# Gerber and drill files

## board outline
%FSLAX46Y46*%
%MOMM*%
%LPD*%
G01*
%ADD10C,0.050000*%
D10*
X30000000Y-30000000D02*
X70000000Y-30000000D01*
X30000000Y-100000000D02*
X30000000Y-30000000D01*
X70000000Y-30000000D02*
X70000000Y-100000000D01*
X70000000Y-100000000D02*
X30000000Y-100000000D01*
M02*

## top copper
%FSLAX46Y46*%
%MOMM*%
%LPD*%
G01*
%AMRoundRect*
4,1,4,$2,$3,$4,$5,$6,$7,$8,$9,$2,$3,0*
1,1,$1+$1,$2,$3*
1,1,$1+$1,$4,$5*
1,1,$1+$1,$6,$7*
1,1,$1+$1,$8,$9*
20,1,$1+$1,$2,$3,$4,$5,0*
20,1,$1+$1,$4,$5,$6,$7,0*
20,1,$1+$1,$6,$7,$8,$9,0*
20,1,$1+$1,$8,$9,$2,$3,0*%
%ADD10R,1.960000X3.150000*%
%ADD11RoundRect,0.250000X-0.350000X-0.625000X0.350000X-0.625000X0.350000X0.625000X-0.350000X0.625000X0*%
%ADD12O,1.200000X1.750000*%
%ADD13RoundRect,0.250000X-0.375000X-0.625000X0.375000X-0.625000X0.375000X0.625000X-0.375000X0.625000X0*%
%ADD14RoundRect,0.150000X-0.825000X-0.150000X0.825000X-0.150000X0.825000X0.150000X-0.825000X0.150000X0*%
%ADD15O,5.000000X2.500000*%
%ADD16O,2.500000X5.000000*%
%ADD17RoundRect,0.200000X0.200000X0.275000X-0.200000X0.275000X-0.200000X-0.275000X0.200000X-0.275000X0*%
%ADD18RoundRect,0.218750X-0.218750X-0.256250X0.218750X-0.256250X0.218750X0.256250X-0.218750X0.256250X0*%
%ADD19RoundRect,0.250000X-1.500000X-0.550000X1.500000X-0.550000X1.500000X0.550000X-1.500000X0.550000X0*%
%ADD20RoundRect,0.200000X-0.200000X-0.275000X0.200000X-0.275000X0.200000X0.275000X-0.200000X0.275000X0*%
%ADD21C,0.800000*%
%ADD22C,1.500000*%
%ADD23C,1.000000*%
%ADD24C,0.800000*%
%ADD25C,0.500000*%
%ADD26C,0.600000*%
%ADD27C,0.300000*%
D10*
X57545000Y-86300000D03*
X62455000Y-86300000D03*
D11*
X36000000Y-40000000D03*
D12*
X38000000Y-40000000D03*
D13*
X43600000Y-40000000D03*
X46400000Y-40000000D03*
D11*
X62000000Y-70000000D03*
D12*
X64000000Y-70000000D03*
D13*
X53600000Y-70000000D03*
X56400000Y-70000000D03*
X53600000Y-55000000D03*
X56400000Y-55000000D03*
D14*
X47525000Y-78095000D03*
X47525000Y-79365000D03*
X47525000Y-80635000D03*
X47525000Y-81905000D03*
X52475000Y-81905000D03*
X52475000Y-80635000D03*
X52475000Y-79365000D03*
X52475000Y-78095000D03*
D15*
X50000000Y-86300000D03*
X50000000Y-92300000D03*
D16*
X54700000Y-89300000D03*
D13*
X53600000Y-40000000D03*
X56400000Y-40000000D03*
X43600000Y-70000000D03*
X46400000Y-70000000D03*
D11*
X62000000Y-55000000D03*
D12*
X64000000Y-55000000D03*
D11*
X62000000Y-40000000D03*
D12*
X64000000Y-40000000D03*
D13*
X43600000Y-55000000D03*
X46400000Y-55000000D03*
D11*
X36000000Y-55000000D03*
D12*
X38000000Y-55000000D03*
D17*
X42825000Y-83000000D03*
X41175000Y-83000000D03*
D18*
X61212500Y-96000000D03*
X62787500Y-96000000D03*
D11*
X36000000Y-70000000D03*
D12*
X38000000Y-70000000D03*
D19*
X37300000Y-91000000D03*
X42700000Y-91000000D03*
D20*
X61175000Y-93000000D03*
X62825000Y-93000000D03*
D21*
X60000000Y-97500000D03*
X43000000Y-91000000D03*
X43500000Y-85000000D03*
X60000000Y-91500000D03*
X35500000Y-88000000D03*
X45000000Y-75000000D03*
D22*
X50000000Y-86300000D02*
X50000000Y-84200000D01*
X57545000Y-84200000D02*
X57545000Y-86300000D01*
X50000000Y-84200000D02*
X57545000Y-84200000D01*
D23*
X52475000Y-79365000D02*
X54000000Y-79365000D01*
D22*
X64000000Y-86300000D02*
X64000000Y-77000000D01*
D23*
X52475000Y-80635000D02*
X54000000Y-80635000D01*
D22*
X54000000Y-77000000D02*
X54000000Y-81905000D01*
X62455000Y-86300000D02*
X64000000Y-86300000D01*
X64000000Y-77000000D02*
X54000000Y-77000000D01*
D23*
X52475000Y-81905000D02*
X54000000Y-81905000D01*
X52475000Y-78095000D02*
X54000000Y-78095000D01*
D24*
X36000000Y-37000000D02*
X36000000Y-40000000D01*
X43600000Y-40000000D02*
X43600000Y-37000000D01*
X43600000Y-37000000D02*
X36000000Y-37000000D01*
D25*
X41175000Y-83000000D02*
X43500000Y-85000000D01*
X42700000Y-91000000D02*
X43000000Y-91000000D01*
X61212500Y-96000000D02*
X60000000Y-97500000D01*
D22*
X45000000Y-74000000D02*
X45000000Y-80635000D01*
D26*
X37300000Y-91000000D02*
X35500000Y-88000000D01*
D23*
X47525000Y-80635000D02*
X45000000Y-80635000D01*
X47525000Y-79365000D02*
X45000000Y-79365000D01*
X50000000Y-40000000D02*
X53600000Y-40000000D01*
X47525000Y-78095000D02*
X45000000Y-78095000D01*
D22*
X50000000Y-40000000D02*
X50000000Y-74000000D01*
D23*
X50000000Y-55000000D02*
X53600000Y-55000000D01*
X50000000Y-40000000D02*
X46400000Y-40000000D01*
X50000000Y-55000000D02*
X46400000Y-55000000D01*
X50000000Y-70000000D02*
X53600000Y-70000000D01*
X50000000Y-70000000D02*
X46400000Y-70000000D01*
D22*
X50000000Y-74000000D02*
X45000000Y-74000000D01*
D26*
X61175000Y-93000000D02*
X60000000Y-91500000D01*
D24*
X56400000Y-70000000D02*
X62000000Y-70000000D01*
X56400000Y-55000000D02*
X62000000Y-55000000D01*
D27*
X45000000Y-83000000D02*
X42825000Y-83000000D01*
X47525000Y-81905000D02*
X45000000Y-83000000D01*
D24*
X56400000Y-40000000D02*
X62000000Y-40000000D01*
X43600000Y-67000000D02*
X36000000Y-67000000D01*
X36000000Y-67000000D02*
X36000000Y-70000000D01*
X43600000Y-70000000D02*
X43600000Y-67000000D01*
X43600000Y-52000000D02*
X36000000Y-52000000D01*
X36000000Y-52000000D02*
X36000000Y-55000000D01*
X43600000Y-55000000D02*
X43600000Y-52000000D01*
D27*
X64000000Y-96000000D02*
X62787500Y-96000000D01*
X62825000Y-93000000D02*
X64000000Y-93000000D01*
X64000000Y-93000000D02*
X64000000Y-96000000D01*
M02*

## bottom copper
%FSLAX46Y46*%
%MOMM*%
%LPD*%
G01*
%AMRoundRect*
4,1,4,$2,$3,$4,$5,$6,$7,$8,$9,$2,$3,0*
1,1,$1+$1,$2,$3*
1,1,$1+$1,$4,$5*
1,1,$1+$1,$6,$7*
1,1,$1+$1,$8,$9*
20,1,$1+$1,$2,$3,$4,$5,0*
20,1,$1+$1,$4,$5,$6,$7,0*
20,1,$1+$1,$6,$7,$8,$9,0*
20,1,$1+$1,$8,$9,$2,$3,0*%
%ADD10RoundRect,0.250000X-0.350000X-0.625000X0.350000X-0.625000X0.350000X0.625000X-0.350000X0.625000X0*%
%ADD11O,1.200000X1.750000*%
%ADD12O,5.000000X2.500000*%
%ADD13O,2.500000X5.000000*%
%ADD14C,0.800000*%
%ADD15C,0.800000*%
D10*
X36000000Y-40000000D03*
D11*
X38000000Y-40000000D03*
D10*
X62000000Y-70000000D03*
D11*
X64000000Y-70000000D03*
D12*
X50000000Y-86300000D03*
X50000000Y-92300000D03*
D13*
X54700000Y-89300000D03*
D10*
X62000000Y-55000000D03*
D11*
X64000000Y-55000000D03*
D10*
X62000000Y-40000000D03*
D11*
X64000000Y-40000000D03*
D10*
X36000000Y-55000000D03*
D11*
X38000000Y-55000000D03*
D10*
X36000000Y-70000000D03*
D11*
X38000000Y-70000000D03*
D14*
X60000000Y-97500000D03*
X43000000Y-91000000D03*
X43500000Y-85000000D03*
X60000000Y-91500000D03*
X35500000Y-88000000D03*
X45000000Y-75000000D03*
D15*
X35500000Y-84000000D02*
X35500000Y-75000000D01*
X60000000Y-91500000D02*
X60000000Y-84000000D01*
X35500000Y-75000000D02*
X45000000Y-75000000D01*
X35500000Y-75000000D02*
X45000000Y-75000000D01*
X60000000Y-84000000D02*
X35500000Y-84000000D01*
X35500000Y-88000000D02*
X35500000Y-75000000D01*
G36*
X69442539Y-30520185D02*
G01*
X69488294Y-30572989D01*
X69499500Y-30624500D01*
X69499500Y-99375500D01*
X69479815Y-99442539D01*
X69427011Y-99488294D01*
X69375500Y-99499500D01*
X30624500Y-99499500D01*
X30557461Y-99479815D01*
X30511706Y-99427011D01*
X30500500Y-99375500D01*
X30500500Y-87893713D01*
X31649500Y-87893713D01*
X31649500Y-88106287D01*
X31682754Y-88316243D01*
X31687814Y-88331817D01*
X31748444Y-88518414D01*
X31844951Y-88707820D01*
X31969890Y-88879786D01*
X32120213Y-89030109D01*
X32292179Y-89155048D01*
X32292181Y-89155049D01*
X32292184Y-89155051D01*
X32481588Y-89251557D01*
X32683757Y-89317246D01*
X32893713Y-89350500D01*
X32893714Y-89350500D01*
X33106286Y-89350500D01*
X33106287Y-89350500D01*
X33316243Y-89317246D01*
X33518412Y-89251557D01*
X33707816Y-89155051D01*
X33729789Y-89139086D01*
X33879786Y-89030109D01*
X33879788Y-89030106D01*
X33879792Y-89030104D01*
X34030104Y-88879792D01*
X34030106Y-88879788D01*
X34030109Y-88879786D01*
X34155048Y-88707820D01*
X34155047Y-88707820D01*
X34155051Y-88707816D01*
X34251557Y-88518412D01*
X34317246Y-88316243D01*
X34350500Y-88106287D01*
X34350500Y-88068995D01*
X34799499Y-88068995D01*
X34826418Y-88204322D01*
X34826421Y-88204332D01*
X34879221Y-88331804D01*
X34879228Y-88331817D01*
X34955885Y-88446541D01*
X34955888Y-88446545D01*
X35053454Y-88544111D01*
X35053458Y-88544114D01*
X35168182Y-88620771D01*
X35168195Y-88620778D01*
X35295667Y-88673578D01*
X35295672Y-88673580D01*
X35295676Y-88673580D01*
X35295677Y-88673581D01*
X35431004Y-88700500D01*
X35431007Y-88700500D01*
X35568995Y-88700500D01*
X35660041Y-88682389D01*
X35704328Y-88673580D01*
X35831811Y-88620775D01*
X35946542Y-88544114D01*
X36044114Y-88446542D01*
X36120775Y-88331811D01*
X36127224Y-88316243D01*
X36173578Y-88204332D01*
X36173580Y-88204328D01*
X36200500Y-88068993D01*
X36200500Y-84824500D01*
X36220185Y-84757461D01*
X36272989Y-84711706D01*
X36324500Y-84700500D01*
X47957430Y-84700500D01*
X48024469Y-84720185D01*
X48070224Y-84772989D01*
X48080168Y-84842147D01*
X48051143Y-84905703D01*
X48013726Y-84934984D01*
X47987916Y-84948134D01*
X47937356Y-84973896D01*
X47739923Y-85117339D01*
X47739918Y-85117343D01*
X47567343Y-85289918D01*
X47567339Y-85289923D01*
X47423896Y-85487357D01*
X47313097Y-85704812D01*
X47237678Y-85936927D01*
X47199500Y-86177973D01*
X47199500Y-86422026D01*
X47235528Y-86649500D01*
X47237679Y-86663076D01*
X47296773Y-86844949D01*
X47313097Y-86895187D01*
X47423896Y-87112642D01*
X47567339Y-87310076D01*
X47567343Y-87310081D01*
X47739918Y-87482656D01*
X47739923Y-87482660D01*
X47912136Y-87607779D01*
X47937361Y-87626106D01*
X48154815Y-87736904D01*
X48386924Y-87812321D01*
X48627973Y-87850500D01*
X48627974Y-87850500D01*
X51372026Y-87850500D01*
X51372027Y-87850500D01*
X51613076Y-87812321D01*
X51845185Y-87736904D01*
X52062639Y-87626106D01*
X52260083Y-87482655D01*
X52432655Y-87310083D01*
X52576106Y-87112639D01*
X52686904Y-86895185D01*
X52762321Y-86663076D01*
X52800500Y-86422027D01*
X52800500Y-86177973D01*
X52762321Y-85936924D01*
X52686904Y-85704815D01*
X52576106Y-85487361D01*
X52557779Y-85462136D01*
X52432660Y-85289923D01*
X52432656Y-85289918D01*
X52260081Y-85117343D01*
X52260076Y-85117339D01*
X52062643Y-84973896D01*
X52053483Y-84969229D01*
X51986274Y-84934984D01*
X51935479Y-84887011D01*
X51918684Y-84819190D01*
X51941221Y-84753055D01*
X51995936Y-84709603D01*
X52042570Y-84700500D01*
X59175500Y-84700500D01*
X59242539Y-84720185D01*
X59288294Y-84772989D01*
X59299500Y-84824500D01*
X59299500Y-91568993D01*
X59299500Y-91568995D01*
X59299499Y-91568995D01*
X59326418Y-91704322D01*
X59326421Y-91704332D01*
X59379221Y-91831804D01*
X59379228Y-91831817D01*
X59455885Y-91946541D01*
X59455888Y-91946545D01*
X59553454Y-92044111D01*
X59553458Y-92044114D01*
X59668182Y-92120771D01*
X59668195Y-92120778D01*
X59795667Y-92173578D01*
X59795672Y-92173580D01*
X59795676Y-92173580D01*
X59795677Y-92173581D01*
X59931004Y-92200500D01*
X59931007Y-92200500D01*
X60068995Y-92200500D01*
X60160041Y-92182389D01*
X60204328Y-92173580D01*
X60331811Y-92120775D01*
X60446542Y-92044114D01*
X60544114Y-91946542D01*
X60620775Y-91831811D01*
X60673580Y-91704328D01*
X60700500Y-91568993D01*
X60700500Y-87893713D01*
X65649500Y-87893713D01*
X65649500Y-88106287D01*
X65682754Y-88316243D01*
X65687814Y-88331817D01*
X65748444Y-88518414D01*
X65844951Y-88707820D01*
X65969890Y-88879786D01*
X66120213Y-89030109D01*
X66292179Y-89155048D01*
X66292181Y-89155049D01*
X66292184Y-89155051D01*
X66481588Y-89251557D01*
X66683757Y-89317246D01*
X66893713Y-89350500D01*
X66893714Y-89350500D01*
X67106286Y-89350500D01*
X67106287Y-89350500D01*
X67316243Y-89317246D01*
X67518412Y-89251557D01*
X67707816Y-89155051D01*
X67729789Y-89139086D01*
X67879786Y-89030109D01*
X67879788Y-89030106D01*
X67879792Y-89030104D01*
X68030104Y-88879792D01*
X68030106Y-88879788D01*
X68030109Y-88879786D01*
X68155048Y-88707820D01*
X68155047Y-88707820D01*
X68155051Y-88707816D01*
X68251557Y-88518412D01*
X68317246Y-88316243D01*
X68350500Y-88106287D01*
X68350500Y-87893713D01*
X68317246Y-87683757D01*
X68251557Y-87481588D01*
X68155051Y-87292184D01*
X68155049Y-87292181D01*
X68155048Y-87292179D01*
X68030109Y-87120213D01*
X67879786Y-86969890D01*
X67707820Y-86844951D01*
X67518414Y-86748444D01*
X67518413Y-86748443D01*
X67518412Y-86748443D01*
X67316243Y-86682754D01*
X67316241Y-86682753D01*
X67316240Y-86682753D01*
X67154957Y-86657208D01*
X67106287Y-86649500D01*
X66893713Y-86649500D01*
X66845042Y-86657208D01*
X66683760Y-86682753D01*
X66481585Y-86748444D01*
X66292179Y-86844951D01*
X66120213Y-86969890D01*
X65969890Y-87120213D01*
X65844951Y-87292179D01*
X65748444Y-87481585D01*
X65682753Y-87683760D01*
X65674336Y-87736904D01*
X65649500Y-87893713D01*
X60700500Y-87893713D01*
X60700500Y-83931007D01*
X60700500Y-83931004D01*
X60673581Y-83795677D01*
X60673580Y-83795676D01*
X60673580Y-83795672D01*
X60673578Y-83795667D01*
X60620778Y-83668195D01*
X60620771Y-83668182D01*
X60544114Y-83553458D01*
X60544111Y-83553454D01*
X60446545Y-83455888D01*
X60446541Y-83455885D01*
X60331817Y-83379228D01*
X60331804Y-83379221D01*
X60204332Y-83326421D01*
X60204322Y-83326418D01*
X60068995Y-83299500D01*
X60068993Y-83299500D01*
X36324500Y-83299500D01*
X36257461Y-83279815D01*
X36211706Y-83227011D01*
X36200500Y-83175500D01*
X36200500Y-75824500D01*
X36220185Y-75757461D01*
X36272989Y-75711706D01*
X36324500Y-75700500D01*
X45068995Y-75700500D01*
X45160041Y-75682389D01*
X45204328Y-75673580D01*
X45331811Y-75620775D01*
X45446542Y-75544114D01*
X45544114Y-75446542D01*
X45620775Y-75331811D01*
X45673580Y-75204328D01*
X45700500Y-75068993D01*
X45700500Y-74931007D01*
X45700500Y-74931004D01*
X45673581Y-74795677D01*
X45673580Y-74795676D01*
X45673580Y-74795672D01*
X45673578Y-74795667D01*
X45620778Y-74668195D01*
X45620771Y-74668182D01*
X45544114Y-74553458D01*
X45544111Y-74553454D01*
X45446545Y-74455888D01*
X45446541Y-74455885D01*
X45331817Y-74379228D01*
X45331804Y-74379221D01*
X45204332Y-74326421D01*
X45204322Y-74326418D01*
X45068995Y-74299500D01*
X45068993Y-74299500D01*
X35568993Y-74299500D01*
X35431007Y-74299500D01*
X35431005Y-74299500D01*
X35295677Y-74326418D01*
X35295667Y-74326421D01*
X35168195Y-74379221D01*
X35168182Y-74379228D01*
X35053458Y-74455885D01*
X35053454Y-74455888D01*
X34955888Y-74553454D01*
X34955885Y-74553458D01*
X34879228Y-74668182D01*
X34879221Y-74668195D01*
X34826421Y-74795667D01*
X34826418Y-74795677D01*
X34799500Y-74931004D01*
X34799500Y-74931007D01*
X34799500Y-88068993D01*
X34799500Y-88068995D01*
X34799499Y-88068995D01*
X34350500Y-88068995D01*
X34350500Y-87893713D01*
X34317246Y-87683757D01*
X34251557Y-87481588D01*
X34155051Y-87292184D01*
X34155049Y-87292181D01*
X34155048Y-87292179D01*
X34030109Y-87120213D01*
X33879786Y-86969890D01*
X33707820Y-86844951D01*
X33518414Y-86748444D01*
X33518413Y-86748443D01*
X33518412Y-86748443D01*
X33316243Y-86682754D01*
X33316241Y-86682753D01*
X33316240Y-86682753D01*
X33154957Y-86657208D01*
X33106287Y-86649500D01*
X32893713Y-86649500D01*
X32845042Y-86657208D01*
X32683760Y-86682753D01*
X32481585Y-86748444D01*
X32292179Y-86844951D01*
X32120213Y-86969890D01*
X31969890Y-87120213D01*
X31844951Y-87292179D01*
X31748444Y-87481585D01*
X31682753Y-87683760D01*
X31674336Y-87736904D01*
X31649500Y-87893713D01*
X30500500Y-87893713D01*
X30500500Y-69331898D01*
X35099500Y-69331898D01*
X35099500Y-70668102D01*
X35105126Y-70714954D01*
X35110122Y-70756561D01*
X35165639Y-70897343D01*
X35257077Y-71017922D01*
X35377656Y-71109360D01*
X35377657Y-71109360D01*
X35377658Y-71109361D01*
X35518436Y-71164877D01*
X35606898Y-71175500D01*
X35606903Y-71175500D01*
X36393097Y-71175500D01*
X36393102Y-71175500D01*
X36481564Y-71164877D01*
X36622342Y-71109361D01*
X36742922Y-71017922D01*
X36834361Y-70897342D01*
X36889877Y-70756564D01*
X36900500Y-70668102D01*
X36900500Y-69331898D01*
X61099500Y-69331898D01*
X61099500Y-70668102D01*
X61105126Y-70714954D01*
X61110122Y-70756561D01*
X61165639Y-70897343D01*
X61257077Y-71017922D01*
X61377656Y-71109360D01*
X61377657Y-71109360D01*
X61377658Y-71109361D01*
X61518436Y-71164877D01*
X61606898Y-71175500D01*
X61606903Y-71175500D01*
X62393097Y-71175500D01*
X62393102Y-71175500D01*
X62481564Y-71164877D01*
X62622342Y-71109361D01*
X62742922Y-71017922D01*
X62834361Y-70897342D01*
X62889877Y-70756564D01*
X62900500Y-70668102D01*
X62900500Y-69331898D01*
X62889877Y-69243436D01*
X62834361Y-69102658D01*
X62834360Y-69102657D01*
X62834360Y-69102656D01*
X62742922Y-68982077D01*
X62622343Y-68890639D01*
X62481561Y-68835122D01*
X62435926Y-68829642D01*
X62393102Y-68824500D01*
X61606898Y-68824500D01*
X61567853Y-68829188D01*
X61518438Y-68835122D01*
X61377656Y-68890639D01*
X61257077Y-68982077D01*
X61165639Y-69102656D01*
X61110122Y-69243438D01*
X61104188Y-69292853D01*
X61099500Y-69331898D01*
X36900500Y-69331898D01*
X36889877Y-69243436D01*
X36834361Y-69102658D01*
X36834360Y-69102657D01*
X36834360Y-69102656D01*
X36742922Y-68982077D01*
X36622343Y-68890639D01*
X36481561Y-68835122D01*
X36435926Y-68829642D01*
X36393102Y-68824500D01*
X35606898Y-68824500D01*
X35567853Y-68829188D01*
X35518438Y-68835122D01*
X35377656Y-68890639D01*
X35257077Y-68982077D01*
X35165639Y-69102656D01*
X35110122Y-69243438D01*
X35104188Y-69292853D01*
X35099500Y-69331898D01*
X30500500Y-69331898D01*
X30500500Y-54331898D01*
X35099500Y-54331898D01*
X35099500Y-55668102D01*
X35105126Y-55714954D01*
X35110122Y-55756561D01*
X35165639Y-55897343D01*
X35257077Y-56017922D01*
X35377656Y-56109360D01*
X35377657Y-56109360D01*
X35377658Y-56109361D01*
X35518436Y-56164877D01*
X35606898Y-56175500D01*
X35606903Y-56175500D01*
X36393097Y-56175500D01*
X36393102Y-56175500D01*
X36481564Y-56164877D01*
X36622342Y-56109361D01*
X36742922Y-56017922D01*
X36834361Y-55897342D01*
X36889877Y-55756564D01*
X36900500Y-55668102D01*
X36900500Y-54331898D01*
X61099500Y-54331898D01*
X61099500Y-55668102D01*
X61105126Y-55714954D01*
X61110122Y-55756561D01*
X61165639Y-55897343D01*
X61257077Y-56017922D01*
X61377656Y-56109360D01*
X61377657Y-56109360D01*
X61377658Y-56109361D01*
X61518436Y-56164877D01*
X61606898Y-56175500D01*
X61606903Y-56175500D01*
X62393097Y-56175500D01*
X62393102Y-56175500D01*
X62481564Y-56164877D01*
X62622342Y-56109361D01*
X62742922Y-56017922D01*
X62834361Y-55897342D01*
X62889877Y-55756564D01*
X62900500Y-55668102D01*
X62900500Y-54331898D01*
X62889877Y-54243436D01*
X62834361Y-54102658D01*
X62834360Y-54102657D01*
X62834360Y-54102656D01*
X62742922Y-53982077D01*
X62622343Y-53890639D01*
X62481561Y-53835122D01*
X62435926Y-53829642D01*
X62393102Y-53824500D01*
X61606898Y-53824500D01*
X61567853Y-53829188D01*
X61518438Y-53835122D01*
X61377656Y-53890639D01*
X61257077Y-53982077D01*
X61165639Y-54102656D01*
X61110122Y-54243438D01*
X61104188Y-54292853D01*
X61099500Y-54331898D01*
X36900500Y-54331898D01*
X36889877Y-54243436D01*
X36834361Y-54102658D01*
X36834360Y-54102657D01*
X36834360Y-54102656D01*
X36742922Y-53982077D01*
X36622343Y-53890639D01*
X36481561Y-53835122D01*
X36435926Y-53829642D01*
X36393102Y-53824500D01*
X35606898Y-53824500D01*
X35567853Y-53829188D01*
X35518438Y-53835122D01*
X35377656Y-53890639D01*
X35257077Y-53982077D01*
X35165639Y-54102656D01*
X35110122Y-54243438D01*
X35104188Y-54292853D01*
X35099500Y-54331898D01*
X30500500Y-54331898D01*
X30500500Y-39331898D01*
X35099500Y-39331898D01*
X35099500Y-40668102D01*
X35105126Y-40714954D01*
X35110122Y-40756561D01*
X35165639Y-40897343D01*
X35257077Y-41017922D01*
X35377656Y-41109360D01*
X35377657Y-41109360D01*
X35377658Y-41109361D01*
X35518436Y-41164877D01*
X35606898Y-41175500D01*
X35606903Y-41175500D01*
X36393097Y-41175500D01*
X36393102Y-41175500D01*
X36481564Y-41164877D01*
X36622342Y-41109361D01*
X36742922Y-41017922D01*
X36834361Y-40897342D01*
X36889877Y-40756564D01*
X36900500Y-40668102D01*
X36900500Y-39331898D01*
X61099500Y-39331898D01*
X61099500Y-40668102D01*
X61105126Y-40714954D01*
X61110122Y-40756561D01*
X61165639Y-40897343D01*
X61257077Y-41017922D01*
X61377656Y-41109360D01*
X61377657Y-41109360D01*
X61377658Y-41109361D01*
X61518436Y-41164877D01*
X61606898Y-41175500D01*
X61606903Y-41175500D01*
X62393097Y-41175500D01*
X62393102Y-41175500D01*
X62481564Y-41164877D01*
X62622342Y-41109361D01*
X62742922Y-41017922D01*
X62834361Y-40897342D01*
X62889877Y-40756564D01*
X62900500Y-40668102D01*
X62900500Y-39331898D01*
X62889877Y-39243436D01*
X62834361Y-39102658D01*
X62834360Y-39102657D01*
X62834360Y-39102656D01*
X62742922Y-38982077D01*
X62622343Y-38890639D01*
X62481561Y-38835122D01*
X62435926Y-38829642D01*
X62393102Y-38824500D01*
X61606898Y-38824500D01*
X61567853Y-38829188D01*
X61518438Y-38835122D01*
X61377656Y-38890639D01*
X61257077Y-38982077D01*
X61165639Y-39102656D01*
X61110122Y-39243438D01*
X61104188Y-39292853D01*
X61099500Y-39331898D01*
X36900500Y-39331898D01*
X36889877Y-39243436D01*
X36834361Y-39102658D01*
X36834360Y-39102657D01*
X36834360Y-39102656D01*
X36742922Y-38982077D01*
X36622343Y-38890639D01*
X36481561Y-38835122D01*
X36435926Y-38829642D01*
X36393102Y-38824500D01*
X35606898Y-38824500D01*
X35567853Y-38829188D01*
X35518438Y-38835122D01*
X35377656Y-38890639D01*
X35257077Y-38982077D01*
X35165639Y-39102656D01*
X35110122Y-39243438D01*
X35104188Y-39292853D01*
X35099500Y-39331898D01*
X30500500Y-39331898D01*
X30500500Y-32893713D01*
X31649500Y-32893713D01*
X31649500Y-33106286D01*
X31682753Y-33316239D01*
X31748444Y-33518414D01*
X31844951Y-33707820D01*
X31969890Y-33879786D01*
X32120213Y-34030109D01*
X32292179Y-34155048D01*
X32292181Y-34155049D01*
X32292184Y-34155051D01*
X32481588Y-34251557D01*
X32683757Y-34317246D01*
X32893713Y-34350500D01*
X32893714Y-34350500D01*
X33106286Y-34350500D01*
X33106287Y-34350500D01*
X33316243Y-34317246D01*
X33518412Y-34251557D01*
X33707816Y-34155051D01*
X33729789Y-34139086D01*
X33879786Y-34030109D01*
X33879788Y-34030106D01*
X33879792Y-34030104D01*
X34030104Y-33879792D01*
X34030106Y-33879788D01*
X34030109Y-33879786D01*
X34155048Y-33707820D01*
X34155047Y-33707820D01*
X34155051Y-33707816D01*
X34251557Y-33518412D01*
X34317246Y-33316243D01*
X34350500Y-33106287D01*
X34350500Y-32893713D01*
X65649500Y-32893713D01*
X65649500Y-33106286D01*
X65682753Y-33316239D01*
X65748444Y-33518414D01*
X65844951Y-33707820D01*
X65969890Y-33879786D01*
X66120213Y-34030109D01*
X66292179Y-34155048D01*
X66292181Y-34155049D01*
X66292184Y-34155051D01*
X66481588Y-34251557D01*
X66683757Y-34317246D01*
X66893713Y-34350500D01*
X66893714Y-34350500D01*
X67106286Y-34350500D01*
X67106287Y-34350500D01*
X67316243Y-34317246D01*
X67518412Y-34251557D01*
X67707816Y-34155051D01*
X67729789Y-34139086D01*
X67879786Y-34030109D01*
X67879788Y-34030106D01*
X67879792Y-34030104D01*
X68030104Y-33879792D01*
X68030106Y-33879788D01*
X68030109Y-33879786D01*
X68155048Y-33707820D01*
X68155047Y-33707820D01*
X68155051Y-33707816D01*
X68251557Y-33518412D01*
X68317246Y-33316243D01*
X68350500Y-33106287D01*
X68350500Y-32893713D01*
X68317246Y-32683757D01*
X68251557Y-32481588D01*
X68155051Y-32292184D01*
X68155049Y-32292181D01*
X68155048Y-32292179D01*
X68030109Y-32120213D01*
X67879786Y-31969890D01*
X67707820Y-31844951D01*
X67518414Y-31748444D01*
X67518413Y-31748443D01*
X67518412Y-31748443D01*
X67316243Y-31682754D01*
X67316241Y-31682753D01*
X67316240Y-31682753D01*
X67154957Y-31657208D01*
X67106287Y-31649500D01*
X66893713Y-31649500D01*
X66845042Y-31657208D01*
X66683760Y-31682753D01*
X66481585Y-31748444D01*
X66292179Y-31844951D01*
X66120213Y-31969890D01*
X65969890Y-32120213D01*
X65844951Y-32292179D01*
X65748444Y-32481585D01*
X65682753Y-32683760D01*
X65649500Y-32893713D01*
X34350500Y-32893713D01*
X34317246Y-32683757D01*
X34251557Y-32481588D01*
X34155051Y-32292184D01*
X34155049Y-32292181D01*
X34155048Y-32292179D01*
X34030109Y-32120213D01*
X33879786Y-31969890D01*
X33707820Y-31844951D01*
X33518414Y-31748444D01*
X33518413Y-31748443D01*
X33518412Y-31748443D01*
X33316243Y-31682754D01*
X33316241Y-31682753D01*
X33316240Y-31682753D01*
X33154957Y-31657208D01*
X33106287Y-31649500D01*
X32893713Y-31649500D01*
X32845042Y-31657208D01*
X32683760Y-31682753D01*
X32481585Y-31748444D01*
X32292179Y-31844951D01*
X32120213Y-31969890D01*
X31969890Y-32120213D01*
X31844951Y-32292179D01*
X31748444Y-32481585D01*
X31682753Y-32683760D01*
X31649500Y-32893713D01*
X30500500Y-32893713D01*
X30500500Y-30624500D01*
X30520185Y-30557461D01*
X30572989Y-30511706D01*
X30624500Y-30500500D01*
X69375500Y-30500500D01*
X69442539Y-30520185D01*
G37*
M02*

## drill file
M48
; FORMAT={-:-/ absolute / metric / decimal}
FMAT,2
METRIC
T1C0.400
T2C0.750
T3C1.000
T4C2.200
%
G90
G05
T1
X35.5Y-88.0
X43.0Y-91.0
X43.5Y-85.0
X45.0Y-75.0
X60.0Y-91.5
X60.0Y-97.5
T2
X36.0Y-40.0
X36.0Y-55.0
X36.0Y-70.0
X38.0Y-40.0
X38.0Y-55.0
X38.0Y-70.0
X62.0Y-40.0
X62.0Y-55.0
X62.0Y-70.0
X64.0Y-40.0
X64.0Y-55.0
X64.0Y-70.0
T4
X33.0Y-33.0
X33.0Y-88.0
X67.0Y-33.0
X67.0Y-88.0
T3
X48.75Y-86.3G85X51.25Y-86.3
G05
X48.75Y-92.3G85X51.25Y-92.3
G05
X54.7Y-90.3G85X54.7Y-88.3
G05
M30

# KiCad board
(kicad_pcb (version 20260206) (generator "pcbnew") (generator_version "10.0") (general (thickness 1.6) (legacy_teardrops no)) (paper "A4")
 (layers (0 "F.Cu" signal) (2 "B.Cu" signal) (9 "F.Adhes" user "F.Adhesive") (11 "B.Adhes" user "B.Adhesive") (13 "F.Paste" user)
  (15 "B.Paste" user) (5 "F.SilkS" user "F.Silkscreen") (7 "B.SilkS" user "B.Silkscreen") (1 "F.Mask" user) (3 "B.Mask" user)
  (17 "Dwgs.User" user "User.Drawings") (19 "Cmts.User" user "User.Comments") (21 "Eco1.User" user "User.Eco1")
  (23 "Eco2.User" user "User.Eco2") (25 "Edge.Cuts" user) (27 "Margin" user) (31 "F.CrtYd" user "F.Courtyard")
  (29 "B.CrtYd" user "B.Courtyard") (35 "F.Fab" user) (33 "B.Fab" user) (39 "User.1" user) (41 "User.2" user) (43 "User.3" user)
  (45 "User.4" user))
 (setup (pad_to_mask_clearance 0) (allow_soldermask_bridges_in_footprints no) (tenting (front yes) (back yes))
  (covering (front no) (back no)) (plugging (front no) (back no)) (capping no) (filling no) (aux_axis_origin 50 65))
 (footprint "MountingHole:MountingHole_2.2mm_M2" (layer "F.Cu") (at 33 88)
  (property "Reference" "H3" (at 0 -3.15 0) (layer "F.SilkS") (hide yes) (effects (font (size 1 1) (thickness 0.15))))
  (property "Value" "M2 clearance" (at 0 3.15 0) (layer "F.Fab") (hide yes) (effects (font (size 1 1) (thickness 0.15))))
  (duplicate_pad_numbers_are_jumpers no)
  (pad "" np_thru_hole circle (at 0 0) (size 2.2 2.2) (drill 2.2) (layers "*.Cu" "*.Mask")))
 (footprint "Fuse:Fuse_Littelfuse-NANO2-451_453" (layer "F.Cu") (at 60 86.3)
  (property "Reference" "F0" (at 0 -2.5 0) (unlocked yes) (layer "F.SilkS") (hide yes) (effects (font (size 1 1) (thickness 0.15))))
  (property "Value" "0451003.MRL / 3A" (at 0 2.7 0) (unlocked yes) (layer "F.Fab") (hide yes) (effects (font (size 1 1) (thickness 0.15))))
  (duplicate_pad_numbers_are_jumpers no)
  (pad "1" smd rect (at -2.455 0) (size 1.96 3.15) (layers "F.Cu" "F.Mask" "F.Paste") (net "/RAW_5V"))
  (pad "2" smd rect (at 2.455 0) (size 1.96 3.15) (layers "F.Cu" "F.Mask" "F.Paste") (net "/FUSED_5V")))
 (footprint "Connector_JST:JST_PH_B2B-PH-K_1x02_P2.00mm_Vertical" (layer "F.Cu") (at 36 40)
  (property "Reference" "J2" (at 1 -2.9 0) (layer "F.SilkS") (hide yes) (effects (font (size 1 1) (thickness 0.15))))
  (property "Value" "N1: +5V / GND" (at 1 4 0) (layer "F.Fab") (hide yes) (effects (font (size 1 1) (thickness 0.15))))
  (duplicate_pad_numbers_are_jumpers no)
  (pad "1" thru_hole roundrect (at 0 0) (size 1.2 1.75) (drill 0.75) (layers "*.Cu" "*.Mask") (remove_unused_layers no)
   (roundrect_rratio 0.208333) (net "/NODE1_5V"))
  (pad "2" thru_hole oval (at 2 0) (size 1.2 1.75) (drill 0.75) (layers "*.Cu" "*.Mask") (remove_unused_layers no) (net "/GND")))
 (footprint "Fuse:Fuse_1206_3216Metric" (layer "F.Cu") (at 45 40)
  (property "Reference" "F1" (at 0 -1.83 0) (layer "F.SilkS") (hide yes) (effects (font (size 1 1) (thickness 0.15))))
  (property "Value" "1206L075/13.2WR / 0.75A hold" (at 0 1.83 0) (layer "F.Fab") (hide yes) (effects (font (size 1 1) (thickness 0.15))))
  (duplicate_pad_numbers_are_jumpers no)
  (pad "1" smd roundrect (at -1.4 0) (size 1.25 1.75) (layers "F.Cu" "F.Mask" "F.Paste") (roundrect_rratio 0.2) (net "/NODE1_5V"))
  (pad "2" smd roundrect (at 1.4 0) (size 1.25 1.75) (layers "F.Cu" "F.Mask" "F.Paste") (roundrect_rratio 0.2) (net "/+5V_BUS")))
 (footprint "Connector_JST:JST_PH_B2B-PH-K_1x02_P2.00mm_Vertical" (layer "F.Cu") (at 62 70)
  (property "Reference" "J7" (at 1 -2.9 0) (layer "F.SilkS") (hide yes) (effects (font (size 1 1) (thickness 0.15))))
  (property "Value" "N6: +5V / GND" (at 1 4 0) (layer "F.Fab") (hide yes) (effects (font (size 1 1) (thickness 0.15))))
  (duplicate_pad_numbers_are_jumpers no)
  (pad "1" thru_hole roundrect (at 0 0) (size 1.2 1.75) (drill 0.75) (layers "*.Cu" "*.Mask") (remove_unused_layers no)
   (roundrect_rratio 0.208333) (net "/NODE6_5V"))
  (pad "2" thru_hole oval (at 2 0) (size 1.2 1.75) (drill 0.75) (layers "*.Cu" "*.Mask") (remove_unused_layers no) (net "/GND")))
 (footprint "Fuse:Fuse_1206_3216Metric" (layer "F.Cu") (at 55 70)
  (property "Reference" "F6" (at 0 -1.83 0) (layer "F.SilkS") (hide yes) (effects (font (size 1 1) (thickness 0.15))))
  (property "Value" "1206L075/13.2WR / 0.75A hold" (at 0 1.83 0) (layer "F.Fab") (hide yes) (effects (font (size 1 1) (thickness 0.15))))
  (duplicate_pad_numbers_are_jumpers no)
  (pad "1" smd roundrect (at -1.4 0) (size 1.25 1.75) (layers "F.Cu" "F.Mask" "F.Paste") (roundrect_rratio 0.2) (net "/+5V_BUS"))
  (pad "2" smd roundrect (at 1.4 0) (size 1.25 1.75) (layers "F.Cu" "F.Mask" "F.Paste") (roundrect_rratio 0.2) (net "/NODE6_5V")))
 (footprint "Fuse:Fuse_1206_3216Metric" (layer "F.Cu") (at 55 55)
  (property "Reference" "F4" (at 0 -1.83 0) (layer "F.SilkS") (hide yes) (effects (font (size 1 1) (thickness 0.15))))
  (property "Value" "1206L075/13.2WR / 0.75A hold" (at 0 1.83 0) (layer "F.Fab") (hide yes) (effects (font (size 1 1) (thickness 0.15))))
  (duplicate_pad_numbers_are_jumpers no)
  (pad "1" smd roundrect (at -1.4 0) (size 1.25 1.75) (layers "F.Cu" "F.Mask" "F.Paste") (roundrect_rratio 0.2) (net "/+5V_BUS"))
  (pad "2" smd roundrect (at 1.4 0) (size 1.25 1.75) (layers "F.Cu" "F.Mask" "F.Paste") (roundrect_rratio 0.2) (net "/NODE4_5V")))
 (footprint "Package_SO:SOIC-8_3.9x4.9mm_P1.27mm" (layer "F.Cu") (at 50 80)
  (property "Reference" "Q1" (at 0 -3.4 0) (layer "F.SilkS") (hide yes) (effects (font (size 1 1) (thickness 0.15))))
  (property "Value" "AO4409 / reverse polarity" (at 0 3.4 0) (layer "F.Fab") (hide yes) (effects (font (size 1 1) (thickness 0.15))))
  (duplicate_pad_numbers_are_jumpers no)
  (pad "1" smd roundrect (at -2.475 -1.905) (size 1.95 0.6) (layers "F.Cu" "F.Mask" "F.Paste") (roundrect_rratio 0.25) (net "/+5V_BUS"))
  (pad "2" smd roundrect (at -2.475 -0.635) (size 1.95 0.6) (layers "F.Cu" "F.Mask" "F.Paste") (roundrect_rratio 0.25) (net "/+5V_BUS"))
  (pad "3" smd roundrect (at -2.475 0.635) (size 1.95 0.6) (layers "F.Cu" "F.Mask" "F.Paste") (roundrect_rratio 0.25) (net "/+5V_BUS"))
  (pad "4" smd roundrect (at -2.475 1.905) (size 1.95 0.6) (layers "F.Cu" "F.Mask" "F.Paste") (roundrect_rratio 0.25) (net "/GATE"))
  (pad "5" smd roundrect (at 2.475 1.905) (size 1.95 0.6) (layers "F.Cu" "F.Mask" "F.Paste") (roundrect_rratio 0.25) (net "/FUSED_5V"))
  (pad "6" smd roundrect (at 2.475 0.635) (size 1.95 0.6) (layers "F.Cu" "F.Mask" "F.Paste") (roundrect_rratio 0.25) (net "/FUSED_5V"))
  (pad "7" smd roundrect (at 2.475 -0.635) (size 1.95 0.6) (layers "F.Cu" "F.Mask" "F.Paste") (roundrect_rratio 0.25) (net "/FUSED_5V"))
  (pad "8" smd roundrect (at 2.475 -1.905) (size 1.95 0.6) (layers "F.Cu" "F.Mask" "F.Paste") (roundrect_rratio 0.25) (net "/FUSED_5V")))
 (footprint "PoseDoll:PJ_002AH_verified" (layer "F.Cu") (at 50 86.3 90)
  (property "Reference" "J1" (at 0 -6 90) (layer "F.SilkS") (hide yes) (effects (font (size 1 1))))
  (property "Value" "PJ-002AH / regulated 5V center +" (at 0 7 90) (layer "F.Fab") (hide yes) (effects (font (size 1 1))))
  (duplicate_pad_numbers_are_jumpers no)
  (pad "1" thru_hole oval (at 0 0 90) (size 2.5 5) (drill oval 1 3.5) (layers "*.Cu" "*.Mask") (remove_unused_layers no) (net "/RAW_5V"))
  (pad "2" thru_hole oval (at -6 0 90) (size 2.5 5) (drill oval 1 3.5) (layers "*.Cu" "*.Mask") (remove_unused_layers no) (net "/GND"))
  (pad "3" thru_hole oval (at -3 4.7 90) (size 5 2.5) (drill oval 3 1) (layers "*.Cu" "*.Mask") (remove_unused_layers no) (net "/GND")))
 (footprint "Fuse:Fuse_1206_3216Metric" (layer "F.Cu") (at 55 40)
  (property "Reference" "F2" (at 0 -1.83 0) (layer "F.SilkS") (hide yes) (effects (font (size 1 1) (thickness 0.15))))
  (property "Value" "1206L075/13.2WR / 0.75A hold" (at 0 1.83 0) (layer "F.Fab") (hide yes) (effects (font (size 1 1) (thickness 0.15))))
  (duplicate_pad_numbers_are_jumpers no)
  (pad "1" smd roundrect (at -1.4 0) (size 1.25 1.75) (layers "F.Cu" "F.Mask" "F.Paste") (roundrect_rratio 0.2) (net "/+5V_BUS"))
  (pad "2" smd roundrect (at 1.4 0) (size 1.25 1.75) (layers "F.Cu" "F.Mask" "F.Paste") (roundrect_rratio 0.2) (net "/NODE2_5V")))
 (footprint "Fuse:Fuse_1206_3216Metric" (layer "F.Cu") (at 45 70)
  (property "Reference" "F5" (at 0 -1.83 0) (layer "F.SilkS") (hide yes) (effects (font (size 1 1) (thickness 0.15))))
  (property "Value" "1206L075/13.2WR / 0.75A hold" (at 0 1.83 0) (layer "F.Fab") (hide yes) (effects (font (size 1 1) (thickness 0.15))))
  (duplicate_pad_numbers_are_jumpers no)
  (pad "1" smd roundrect (at -1.4 0) (size 1.25 1.75) (layers "F.Cu" "F.Mask" "F.Paste") (roundrect_rratio 0.2) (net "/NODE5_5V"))
  (pad "2" smd roundrect (at 1.4 0) (size 1.25 1.75) (layers "F.Cu" "F.Mask" "F.Paste") (roundrect_rratio 0.2) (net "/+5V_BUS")))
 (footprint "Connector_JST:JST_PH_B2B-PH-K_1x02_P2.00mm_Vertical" (layer "F.Cu") (at 62 55)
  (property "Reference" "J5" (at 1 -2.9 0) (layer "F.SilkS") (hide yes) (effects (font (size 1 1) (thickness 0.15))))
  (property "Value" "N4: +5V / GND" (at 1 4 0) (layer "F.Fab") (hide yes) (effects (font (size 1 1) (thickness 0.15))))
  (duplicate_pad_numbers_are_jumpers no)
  (pad "1" thru_hole roundrect (at 0 0) (size 1.2 1.75) (drill 0.75) (layers "*.Cu" "*.Mask") (remove_unused_layers no)
   (roundrect_rratio 0.208333) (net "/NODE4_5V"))
  (pad "2" thru_hole oval (at 2 0) (size 1.2 1.75) (drill 0.75) (layers "*.Cu" "*.Mask") (remove_unused_layers no) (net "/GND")))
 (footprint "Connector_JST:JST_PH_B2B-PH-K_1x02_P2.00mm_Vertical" (layer "F.Cu") (at 62 40)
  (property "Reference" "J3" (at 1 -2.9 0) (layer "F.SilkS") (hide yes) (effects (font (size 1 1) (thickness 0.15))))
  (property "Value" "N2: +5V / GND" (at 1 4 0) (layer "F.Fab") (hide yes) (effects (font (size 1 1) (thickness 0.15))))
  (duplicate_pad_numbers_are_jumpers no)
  (pad "1" thru_hole roundrect (at 0 0) (size 1.2 1.75) (drill 0.75) (layers "*.Cu" "*.Mask") (remove_unused_layers no)
   (roundrect_rratio 0.208333) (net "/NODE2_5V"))
  (pad "2" thru_hole oval (at 2 0) (size 1.2 1.75) (drill 0.75) (layers "*.Cu" "*.Mask") (remove_unused_layers no) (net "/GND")))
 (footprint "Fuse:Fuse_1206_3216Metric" (layer "F.Cu") (at 45 55)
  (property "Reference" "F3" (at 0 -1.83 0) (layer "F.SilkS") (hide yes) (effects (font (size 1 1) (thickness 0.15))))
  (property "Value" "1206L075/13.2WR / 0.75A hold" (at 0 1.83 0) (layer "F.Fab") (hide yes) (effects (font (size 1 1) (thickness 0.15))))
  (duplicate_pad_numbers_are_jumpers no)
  (pad "1" smd roundrect (at -1.4 0) (size 1.25 1.75) (layers "F.Cu" "F.Mask" "F.Paste") (roundrect_rratio 0.2) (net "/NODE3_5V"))
  (pad "2" smd roundrect (at 1.4 0) (size 1.25 1.75) (layers "F.Cu" "F.Mask" "F.Paste") (roundrect_rratio 0.2) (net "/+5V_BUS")))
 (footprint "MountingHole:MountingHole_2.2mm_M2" (layer "F.Cu") (at 67 88)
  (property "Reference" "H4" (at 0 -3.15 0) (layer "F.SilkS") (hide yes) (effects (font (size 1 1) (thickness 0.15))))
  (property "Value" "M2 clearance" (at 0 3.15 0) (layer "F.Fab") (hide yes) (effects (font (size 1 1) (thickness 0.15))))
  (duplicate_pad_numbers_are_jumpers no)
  (pad "" np_thru_hole circle (at 0 0) (size 2.2 2.2) (drill 2.2) (layers "*.Cu" "*.Mask")))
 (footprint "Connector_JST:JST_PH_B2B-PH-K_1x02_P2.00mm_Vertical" (layer "F.Cu") (at 36 55)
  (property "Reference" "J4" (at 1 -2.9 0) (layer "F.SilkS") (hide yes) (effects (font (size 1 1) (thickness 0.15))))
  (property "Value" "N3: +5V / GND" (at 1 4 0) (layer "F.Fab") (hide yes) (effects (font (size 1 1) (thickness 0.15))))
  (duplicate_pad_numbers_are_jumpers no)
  (pad "1" thru_hole roundrect (at 0 0) (size 1.2 1.75) (drill 0.75) (layers "*.Cu" "*.Mask") (remove_unused_layers no)
   (roundrect_rratio 0.208333) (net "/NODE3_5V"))
  (pad "2" thru_hole oval (at 2 0) (size 1.2 1.75) (drill 0.75) (layers "*.Cu" "*.Mask") (remove_unused_layers no) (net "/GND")))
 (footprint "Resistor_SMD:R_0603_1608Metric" (layer "F.Cu") (at 42 83 180)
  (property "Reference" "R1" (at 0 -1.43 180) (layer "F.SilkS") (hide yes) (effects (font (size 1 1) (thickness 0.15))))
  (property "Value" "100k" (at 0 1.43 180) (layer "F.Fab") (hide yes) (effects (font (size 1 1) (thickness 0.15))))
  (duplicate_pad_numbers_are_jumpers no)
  (pad "1" smd roundrect (at -0.825 0 180) (size 0.8 0.95) (layers "F.Cu" "F.Mask" "F.Paste") (roundrect_rratio 0.25) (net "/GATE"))
  (pad "2" smd roundrect (at 0.825 0 180) (size 0.8 0.95) (layers "F.Cu" "F.Mask" "F.Paste") (roundrect_rratio 0.25) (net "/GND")))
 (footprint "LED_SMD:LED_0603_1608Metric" (layer "F.Cu") (at 62 96)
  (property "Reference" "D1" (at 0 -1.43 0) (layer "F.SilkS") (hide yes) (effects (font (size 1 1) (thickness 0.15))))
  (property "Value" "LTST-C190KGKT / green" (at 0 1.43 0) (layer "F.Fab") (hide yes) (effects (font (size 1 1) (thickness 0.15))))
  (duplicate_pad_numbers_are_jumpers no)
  (pad "1" smd roundrect (at -0.7875 0) (size 0.875 0.95) (layers "F.Cu" "F.Mask" "F.Paste") (roundrect_rratio 0.25) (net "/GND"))
  (pad "2" smd roundrect (at 0.7875 0) (size 0.875 0.95) (layers "F.Cu" "F.Mask" "F.Paste") (roundrect_rratio 0.25) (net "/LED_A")))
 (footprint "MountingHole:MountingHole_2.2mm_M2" (layer "F.Cu") (at 67 33)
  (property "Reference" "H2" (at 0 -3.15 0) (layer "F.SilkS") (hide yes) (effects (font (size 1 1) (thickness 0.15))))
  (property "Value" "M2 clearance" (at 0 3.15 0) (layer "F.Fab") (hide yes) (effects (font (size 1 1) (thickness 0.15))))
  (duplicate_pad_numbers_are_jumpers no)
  (pad "" np_thru_hole circle (at 0 0) (size 2.2 2.2) (drill 2.2) (layers "*.Cu" "*.Mask")))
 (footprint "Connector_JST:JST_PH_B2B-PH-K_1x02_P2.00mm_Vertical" (layer "F.Cu") (at 36 70)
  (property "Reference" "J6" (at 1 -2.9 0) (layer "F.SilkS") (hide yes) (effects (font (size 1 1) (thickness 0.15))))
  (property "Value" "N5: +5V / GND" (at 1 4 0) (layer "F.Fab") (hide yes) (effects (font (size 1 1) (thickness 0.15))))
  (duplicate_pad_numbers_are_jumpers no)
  (pad "1" thru_hole roundrect (at 0 0) (size 1.2 1.75) (drill 0.75) (layers "*.Cu" "*.Mask") (remove_unused_layers no)
   (roundrect_rratio 0.208333) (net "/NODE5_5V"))
  (pad "2" thru_hole oval (at 2 0) (size 1.2 1.75) (drill 0.75) (layers "*.Cu" "*.Mask") (remove_unused_layers no) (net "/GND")))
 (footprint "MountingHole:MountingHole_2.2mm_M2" (layer "F.Cu") (at 33 33)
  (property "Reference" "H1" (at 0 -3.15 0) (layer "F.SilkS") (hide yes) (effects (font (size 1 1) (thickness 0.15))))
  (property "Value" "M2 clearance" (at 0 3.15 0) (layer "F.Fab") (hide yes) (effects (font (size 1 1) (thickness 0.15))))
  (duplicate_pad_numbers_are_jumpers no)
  (pad "" np_thru_hole circle (at 0 0) (size 2.2 2.2) (drill 2.2) (layers "*.Cu" "*.Mask")))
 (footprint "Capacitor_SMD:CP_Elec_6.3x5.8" (layer "F.Cu") (at 40 91)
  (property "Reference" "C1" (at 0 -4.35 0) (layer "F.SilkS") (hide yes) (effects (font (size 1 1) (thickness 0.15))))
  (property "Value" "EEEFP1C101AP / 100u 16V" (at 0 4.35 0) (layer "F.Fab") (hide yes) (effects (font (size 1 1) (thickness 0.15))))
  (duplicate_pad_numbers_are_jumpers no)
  (pad "1" smd roundrect (at -2.7 0) (size 3.5 1.6) (layers "F.Cu" "F.Mask" "F.Paste") (roundrect_rratio 0.15625) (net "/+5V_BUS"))
  (pad "2" smd roundrect (at 2.7 0) (size 3.5 1.6) (layers "F.Cu" "F.Mask" "F.Paste") (roundrect_rratio 0.15625) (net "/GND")))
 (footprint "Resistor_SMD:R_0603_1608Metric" (layer "F.Cu") (at 62 93)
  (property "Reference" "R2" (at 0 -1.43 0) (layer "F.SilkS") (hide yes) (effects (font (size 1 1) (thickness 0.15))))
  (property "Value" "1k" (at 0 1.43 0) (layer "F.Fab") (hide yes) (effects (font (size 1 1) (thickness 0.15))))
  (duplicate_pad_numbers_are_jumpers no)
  (pad "1" smd roundrect (at -0.825 0) (size 0.8 0.95) (layers "F.Cu" "F.Mask" "F.Paste") (roundrect_rratio 0.25) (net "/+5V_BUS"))
  (pad "2" smd roundrect (at 0.825 0) (size 0.8 0.95) (layers "F.Cu" "F.Mask" "F.Paste") (roundrect_rratio 0.25) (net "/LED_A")))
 (gr_line (start 30 30) (end 70 30) (stroke (width 0.05) (type default)) (layer "Edge.Cuts"))
 (gr_line (start 30 100) (end 30 30) (stroke (width 0.05) (type default)) (layer "Edge.Cuts"))
 (gr_line (start 70 30) (end 70 100) (stroke (width 0.05) (type default)) (layer "Edge.Cuts"))
 (gr_line (start 70 100) (end 30 100) (stroke (width 0.05) (type default)) (layer "Edge.Cuts"))
 (segment (start 50 86.3) (end 50 84.2) (width 1.5) (layer "F.Cu") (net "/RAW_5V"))
 (segment (start 57.545 84.2) (end 57.545 86.3) (width 1.5) (layer "F.Cu") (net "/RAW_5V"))
 (segment (start 50 84.2) (end 57.545 84.2) (width 1.5) (layer "F.Cu") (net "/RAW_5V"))
 (segment (start 52.475 79.365) (end 54 79.365) (width 1) (layer "F.Cu") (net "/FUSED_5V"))
 (segment (start 64 86.3) (end 64 77) (width 1.5) (layer "F.Cu") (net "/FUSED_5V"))
 (segment (start 52.475 80.635) (end 54 80.635) (width 1) (layer "F.Cu") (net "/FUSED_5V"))
 (segment (start 54 77) (end 54 81.905) (width 1.5) (layer "F.Cu") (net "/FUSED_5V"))
 (segment (start 62.455 86.3) (end 64 86.3) (width 1.5) (layer "F.Cu") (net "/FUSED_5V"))
 (segment (start 64 77) (end 54 77) (width 1.5) (layer "F.Cu") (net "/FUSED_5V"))
 (segment (start 52.475 81.905) (end 54 81.905) (width 1) (layer "F.Cu") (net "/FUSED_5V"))
 (segment (start 52.475 78.095) (end 54 78.095) (width 1) (layer "F.Cu") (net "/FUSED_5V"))
 (segment (start 36 37) (end 36 40) (width 0.8) (layer "F.Cu") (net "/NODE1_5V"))
 (segment (start 43.6 40) (end 43.6 37) (width 0.8) (layer "F.Cu") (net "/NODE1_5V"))
 (segment (start 43.6 37) (end 36 37) (width 0.8) (layer "F.Cu") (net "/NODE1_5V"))
 (segment (start 41.175 83) (end 43.5 85) (width 0.5) (layer "F.Cu") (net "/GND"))
 (segment (start 42.7 91) (end 43 91) (width 0.5) (layer "F.Cu") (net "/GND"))
 (segment (start 61.2125 96) (end 60 97.5) (width 0.5) (layer "F.Cu") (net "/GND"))
 (via (at 60 97.5) (size 0.8) (drill 0.4) (layers "F.Cu" "B.Cu") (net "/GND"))
 (via (at 43 91) (size 0.8) (drill 0.4) (layers "F.Cu" "B.Cu") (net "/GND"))
 (via (at 43.5 85) (size 0.8) (drill 0.4) (layers "F.Cu" "B.Cu") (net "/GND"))
 (segment (start 45 74) (end 45 80.635) (width 1.5) (layer "F.Cu") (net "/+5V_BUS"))
 (segment (start 37.3 91) (end 35.5 88) (width 0.6) (layer "F.Cu") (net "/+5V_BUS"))
 (segment (start 47.525 80.635) (end 45 80.635) (width 1) (layer "F.Cu") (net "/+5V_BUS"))
 (segment (start 47.525 79.365) (end 45 79.365) (width 1) (layer "F.Cu") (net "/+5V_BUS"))
 (segment (start 50 40) (end 53.6 40) (width 1) (layer "F.Cu") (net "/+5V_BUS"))
 (segment (start 47.525 78.095) (end 45 78.095) (width 1) (layer "F.Cu") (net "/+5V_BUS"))
 (segment (start 50 40) (end 50 74) (width 1.5) (layer "F.Cu") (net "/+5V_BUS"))
 (segment (start 50 55) (end 53.6 55) (width 1) (layer "F.Cu") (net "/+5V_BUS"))
 (segment (start 50 40) (end 46.4 40) (width 1) (layer "F.Cu") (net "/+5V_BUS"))
 (segment (start 50 55) (end 46.4 55) (width 1) (layer "F.Cu") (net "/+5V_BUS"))
 (segment (start 50 70) (end 53.6 70) (width 1) (layer "F.Cu") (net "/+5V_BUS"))
 (segment (start 50 70) (end 46.4 70) (width 1) (layer "F.Cu") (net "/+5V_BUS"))
 (segment (start 50 74) (end 45 74) (width 1.5) (layer "F.Cu") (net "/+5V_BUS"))
 (segment (start 61.175 93) (end 60 91.5) (width 0.6) (layer "F.Cu") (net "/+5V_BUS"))
 (via (at 60 91.5) (size 0.8) (drill 0.4) (layers "F.Cu" "B.Cu") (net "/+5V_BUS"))
 (via (at 35.5 88) (size 0.8) (drill 0.4) (layers "F.Cu" "B.Cu") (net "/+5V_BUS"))
 (via (at 45 75) (size 0.8) (drill 0.4) (layers "F.Cu" "B.Cu") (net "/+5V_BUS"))
 (segment (start 35.5 84) (end 35.5 75) (width 0.8) (layer "B.Cu") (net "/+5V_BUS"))
 (segment (start 60 91.5) (end 60 84) (width 0.8) (layer "B.Cu") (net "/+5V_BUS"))
 (segment (start 35.5 75) (end 45 75) (width 0.8) (layer "B.Cu") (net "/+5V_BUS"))
 (segment (start 35.5 75) (end 45 75) (width 0.8) (layer "B.Cu") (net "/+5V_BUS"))
 (segment (start 60 84) (end 35.5 84) (width 0.8) (layer "B.Cu") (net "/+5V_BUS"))
 (segment (start 35.5 88) (end 35.5 75) (width 0.8) (layer "B.Cu") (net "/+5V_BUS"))
 (segment (start 56.4 70) (end 62 70) (width 0.8) (layer "F.Cu") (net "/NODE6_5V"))
 (segment (start 56.4 55) (end 62 55) (width 0.8) (layer "F.Cu") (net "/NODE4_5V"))
 (segment (start 45 83) (end 42.825 83) (width 0.3) (layer "F.Cu") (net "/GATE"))
 (segment (start 47.525 81.905) (end 45 83) (width 0.3) (layer "F.Cu") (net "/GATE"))
 (segment (start 56.4 40) (end 62 40) (width 0.8) (layer "F.Cu") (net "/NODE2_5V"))
 (segment (start 43.6 67) (end 36 67) (width 0.8) (layer "F.Cu") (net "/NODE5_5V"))
 (segment (start 36 67) (end 36 70) (width 0.8) (layer "F.Cu") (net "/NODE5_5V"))
 (segment (start 43.6 70) (end 43.6 67) (width 0.8) (layer "F.Cu") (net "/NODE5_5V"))
 (segment (start 43.6 52) (end 36 52) (width 0.8) (layer "F.Cu") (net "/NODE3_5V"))
 (segment (start 36 52) (end 36 55) (width 0.8) (layer "F.Cu") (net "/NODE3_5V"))
 (segment (start 43.6 55) (end 43.6 52) (width 0.8) (layer "F.Cu") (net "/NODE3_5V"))
 (segment (start 64 96) (end 62.7875 96) (width 0.3) (layer "F.Cu") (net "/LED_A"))
 (segment (start 62.825 93) (end 64 93) (width 0.3) (layer "F.Cu") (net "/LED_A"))
 (segment (start 64 93) (end 64 96) (width 0.3) (layer "F.Cu") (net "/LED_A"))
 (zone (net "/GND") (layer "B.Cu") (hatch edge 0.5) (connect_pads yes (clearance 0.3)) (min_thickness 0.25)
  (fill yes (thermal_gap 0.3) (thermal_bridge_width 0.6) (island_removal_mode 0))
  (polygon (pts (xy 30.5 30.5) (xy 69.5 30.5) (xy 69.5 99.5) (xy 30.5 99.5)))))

